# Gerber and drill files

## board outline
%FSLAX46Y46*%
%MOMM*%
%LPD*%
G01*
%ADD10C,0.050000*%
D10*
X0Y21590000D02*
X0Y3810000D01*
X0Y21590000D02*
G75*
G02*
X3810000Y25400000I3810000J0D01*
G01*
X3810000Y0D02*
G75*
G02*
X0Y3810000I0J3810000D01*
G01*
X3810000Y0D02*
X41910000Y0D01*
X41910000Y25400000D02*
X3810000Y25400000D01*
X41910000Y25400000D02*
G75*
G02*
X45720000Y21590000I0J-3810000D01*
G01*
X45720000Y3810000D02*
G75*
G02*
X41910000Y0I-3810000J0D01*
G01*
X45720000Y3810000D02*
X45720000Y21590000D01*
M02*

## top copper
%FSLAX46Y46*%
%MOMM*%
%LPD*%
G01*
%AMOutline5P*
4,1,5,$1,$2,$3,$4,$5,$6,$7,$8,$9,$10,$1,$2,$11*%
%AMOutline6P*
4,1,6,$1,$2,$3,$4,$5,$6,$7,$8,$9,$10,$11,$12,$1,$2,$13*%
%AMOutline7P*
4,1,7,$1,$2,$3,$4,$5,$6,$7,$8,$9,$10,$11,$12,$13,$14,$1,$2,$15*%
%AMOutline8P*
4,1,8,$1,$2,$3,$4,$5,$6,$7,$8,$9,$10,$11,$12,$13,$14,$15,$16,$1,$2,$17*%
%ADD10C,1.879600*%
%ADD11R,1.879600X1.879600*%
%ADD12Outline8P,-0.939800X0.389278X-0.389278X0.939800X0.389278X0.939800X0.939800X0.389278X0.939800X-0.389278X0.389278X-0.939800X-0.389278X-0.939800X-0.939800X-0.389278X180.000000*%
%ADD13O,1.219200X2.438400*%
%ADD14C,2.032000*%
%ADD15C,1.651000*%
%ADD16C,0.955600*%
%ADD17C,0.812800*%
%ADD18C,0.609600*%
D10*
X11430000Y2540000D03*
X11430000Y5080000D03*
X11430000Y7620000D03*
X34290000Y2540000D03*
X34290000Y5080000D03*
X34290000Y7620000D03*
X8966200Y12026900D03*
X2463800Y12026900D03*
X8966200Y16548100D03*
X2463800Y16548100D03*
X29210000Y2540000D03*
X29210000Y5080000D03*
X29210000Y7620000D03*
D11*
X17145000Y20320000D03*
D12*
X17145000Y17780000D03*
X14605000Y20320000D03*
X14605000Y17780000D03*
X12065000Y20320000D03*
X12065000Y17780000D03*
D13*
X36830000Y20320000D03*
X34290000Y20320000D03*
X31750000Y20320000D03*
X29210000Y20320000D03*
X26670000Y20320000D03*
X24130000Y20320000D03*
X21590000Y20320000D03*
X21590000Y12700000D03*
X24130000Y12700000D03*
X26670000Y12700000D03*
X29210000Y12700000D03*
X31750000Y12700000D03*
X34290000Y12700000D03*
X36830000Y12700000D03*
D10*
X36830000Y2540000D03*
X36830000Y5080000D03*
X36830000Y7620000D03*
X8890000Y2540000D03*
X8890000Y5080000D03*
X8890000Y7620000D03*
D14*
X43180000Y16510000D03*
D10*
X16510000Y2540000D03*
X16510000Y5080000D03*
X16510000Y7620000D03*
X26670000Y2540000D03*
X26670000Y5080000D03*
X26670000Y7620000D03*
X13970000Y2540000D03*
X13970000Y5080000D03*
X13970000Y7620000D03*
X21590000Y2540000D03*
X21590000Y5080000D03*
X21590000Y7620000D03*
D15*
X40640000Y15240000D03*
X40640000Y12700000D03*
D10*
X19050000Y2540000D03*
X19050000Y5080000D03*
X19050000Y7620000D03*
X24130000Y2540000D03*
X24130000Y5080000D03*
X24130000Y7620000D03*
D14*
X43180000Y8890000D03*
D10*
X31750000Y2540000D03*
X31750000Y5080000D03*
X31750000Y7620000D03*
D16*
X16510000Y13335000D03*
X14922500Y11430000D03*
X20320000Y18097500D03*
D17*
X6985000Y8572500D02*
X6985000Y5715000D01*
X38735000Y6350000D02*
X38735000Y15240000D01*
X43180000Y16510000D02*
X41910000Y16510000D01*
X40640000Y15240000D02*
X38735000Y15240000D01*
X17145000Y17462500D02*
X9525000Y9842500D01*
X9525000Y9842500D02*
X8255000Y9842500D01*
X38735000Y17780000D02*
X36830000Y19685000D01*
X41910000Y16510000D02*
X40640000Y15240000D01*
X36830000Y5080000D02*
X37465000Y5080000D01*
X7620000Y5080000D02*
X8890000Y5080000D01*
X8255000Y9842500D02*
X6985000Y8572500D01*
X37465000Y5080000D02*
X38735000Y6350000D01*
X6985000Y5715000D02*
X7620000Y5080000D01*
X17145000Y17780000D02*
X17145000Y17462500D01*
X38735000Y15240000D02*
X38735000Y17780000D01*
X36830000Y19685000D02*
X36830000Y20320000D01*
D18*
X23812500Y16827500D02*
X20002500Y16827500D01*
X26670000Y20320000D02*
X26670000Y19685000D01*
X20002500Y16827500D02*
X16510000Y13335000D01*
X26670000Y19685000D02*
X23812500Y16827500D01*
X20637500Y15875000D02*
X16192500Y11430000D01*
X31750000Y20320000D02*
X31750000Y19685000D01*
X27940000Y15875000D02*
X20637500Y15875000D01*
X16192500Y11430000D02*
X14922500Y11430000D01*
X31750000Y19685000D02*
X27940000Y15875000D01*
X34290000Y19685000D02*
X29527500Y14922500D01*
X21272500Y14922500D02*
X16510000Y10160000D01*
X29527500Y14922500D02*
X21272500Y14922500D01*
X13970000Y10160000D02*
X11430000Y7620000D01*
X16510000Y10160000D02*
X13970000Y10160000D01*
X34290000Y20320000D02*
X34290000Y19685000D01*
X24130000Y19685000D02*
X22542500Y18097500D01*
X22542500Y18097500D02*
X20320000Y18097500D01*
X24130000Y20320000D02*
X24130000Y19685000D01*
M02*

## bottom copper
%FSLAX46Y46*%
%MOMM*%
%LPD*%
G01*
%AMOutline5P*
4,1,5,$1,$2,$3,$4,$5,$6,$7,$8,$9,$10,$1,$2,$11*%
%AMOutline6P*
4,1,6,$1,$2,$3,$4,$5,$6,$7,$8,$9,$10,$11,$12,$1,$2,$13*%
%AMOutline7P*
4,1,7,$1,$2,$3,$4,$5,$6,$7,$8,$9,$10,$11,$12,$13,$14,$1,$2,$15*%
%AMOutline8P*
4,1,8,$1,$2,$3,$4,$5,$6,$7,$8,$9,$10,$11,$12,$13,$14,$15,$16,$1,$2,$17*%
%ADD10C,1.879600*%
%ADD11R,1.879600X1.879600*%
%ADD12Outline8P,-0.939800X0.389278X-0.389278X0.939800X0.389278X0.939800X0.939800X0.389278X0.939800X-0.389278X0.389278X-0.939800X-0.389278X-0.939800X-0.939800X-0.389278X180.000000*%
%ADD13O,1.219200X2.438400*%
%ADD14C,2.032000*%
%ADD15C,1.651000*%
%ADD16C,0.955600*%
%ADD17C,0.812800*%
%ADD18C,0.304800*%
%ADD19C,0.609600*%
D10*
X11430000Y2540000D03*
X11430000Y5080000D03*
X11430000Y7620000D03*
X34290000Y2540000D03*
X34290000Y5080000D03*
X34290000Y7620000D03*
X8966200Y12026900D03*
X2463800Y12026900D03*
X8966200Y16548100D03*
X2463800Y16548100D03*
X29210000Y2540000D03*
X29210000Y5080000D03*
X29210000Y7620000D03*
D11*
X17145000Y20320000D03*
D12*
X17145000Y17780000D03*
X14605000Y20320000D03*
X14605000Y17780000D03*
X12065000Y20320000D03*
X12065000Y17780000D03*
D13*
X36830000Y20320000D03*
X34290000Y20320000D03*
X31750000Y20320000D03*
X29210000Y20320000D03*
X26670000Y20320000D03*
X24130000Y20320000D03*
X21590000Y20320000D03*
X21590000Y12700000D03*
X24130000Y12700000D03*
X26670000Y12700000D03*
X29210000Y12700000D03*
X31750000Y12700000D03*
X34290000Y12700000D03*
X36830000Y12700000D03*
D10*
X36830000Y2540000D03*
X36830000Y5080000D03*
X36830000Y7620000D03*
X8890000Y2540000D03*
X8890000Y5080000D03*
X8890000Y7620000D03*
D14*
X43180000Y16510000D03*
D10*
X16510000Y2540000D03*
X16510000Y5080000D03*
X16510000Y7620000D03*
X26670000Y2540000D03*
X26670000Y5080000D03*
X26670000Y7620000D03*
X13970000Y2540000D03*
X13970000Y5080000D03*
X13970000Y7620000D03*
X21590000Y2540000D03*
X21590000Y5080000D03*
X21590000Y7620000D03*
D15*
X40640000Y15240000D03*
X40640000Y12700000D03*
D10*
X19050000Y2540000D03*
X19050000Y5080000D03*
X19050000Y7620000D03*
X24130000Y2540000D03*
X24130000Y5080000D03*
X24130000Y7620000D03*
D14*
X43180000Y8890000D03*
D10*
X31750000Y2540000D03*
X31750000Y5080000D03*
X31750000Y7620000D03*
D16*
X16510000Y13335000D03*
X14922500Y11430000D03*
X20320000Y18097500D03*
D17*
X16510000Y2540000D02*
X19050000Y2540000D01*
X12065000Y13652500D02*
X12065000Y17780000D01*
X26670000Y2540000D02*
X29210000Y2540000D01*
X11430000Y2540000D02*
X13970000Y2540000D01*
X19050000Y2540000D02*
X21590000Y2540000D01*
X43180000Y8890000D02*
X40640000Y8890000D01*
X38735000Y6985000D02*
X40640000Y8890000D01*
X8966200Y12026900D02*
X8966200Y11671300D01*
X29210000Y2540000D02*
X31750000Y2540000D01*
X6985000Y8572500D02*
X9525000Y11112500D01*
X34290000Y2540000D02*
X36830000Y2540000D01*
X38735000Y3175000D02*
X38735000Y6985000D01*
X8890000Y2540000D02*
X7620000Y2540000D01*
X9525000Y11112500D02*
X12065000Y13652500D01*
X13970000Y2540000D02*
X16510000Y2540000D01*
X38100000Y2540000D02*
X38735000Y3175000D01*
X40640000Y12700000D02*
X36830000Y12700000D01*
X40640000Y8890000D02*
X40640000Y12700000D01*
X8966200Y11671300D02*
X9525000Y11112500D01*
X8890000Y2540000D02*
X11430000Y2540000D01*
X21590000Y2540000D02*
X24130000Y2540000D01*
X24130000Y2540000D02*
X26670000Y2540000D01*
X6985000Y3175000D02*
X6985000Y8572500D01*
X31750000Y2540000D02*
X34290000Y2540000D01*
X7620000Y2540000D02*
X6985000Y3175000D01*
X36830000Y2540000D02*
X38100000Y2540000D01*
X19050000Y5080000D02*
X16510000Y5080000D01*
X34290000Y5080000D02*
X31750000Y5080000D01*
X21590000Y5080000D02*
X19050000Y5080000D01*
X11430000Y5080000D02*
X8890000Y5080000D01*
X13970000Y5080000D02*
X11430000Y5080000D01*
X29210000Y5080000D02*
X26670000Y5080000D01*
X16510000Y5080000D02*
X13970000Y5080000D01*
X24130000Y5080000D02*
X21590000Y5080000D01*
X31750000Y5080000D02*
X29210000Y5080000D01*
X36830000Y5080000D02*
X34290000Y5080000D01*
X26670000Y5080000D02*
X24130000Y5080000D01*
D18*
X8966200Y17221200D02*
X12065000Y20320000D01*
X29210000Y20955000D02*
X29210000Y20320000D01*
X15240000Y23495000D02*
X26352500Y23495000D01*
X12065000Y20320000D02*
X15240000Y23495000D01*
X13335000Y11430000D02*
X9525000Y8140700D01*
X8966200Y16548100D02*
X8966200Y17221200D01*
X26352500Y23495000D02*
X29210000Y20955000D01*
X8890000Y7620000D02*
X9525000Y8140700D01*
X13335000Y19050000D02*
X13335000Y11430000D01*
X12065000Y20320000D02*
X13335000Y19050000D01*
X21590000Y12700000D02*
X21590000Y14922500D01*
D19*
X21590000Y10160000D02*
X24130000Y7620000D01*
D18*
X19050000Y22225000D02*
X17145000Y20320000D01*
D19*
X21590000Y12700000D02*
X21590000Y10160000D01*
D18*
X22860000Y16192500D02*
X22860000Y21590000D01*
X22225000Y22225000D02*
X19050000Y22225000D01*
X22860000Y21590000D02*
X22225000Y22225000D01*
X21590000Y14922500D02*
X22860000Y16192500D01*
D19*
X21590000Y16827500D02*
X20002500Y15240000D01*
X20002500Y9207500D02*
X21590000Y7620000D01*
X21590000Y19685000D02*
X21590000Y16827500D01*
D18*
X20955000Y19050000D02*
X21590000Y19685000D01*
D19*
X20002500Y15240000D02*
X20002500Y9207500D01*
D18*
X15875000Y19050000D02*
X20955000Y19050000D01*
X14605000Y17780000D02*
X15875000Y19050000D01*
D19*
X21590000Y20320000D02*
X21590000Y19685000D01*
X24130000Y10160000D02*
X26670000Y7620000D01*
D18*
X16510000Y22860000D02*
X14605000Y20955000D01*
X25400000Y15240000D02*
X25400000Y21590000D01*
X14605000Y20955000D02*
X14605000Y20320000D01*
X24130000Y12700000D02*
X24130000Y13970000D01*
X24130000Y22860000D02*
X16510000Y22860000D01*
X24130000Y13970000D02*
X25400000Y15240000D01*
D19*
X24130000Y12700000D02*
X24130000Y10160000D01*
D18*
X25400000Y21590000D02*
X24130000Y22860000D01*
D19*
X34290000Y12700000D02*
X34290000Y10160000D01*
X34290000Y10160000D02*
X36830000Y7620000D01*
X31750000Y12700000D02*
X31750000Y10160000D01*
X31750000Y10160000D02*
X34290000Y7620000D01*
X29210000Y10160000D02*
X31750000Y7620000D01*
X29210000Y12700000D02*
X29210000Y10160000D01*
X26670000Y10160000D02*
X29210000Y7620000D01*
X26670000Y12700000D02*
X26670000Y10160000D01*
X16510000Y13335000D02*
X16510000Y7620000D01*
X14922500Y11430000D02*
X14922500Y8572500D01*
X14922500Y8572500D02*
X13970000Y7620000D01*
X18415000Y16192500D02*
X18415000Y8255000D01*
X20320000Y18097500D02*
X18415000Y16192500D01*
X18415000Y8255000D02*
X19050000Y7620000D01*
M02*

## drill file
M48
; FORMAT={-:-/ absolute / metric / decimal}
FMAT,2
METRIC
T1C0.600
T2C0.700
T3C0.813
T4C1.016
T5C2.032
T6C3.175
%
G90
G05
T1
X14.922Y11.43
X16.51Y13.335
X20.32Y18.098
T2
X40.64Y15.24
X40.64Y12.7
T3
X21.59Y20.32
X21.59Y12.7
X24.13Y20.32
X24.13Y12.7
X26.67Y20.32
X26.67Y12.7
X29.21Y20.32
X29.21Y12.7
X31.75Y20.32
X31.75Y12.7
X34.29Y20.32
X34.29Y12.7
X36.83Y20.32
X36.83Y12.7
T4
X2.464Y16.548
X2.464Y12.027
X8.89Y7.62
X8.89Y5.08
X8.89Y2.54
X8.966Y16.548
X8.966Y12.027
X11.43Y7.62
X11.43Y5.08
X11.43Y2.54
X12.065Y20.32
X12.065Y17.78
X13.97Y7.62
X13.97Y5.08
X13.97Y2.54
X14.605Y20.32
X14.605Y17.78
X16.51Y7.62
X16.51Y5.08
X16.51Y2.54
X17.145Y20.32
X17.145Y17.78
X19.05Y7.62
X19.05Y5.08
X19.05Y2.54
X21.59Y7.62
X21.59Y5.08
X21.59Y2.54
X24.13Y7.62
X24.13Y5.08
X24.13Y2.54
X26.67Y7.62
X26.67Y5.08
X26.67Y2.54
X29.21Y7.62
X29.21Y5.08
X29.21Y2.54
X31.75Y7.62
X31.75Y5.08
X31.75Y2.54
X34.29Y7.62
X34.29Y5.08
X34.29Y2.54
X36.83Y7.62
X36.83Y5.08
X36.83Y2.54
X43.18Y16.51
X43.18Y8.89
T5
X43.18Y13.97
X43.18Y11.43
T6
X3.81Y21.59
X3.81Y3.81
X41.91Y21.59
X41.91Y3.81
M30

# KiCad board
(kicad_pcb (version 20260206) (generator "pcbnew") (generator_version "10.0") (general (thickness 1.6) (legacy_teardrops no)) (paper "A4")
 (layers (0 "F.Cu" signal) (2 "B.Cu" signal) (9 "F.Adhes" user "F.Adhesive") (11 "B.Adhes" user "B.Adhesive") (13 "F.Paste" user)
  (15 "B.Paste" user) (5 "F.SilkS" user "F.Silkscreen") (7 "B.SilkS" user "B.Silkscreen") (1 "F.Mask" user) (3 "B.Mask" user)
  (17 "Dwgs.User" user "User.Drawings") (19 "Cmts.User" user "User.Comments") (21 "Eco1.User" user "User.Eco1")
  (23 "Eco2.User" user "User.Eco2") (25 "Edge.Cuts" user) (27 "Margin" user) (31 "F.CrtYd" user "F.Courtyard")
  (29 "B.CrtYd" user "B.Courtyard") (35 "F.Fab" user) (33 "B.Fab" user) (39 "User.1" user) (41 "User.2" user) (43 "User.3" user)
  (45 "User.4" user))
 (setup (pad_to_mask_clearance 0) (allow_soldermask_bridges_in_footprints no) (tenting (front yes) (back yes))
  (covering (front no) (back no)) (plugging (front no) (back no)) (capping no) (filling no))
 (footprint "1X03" (layer "F.Cu") (at 11.43 -2.54 90)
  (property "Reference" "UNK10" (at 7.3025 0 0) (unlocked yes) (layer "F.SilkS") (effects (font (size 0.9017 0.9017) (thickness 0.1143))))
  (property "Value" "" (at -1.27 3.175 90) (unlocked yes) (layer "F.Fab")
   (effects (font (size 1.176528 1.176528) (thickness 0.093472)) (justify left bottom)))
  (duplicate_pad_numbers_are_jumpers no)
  (pad "1" thru_hole circle (at 0 0 180) (size 1.8796 1.8796) (drill 1.016) (layers "*.Cu" "*.Mask") (remove_unused_layers no) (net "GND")
   (solder_mask_margin 0.0762) (thermal_bridge_angle 0))
  (pad "2" thru_hole circle (at 2.54 0 180) (size 1.8796 1.8796) (drill 1.016) (layers "*.Cu" "*.Mask") (remove_unused_layers no)
   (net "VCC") (solder_mask_margin 0.0762) (thermal_bridge_angle 0))
  (pad "3" thru_hole circle (at 5.08 0 180) (size 1.8796 1.8796) (drill 1.016) (layers "*.Cu" "*.Mask") (remove_unused_layers no)
   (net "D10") (solder_mask_margin 0.0762) (thermal_bridge_angle 0)))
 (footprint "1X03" (layer "F.Cu") (at 34.29 -2.54 90)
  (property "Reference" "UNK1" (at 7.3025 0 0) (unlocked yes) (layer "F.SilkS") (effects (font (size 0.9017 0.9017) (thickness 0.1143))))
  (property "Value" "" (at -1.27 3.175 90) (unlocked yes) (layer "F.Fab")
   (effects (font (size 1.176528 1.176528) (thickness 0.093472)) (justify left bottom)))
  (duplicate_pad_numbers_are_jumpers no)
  (pad "1" thru_hole circle (at 0 0 180) (size 1.8796 1.8796) (drill 1.016) (layers "*.Cu" "*.Mask") (remove_unused_layers no) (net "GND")
   (solder_mask_margin 0.0762) (thermal_bridge_angle 0))
  (pad "2" thru_hole circle (at 2.54 0 180) (size 1.8796 1.8796) (drill 1.016) (layers "*.Cu" "*.Mask") (remove_unused_layers no)
   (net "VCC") (solder_mask_margin 0.0762) (thermal_bridge_angle 0))
  (pad "3" thru_hole circle (at 5.08 0 180) (size 1.8796 1.8796) (drill 1.016) (layers "*.Cu" "*.Mask") (remove_unused_layers no) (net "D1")
   (solder_mask_margin 0.0762) (thermal_bridge_angle 0)))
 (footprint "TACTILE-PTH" (layer "F.Cu") (at 5.715 -14.2875 180)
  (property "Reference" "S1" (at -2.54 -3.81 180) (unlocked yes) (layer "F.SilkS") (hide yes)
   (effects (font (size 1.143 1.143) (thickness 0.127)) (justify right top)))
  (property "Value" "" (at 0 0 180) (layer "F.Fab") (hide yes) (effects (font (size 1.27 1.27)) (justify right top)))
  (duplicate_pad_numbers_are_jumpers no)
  (pad "1" thru_hole circle (at -3.2512 -2.2606 180) (size 1.8796 1.8796) (drill 1.016) (layers "*.Cu" "*.Mask") (remove_unused_layers no)
   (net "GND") (solder_mask_margin 0.0762) (thermal_bridge_angle 0))
  (pad "2" thru_hole circle (at 3.2512 -2.2606 180) (size 1.8796 1.8796) (drill 1.016) (layers "*.Cu" "*.Mask") (remove_unused_layers no)
   (solder_mask_margin 0.0762) (thermal_bridge_angle 0))
  (pad "3" thru_hole circle (at -3.2512 2.2606 180) (size 1.8796 1.8796) (drill 1.016) (layers "*.Cu" "*.Mask") (remove_unused_layers no)
   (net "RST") (solder_mask_margin 0.0762) (thermal_bridge_angle 0))
  (pad "4" thru_hole circle (at 3.2512 2.2606 180) (size 1.8796 1.8796) (drill 1.016) (layers "*.Cu" "*.Mask") (remove_unused_layers no)
   (solder_mask_margin 0.0762) (thermal_bridge_angle 0)))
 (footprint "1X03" (layer "F.Cu") (at 29.21 -2.54 90)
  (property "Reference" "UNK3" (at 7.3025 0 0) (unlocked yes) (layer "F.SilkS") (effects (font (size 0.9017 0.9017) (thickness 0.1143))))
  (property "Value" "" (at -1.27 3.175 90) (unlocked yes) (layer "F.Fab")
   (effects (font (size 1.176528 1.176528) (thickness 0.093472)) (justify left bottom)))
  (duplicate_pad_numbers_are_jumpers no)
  (pad "1" thru_hole circle (at 0 0 180) (size 1.8796 1.8796) (drill 1.016) (layers "*.Cu" "*.Mask") (remove_unused_layers no) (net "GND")
   (solder_mask_margin 0.0762) (thermal_bridge_angle 0))
  (pad "2" thru_hole circle (at 2.54 0 180) (size 1.8796 1.8796) (drill 1.016) (layers "*.Cu" "*.Mask") (remove_unused_layers no)
   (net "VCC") (solder_mask_margin 0.0762) (thermal_bridge_angle 0))
  (pad "3" thru_hole circle (at 5.08 0 180) (size 1.8796 1.8796) (drill 1.016) (layers "*.Cu" "*.Mask") (remove_unused_layers no) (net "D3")
   (solder_mask_margin 0.0762) (thermal_bridge_angle 0)))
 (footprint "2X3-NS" (layer "F.Cu") (at 14.605 -19.05 180)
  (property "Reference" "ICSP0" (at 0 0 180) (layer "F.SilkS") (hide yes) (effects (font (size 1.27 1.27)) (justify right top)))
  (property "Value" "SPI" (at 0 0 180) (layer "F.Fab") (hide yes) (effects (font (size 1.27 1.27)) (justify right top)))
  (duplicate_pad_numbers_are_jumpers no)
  (pad "1" thru_hole rect (at -2.54 1.27 180) (size 1.8796 1.8796) (drill 1.016) (layers "*.Cu" "*.Mask") (remove_unused_layers no)
   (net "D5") (solder_mask_margin 0.0762) (thermal_bridge_angle 0))
  (pad "2" thru_hole roundrect (at -2.54 -1.27 180) (size 1.8796 1.8796) (drill 1.016) (layers "*.Cu" "*.Mask") (remove_unused_layers no)
   (roundrect_rratio 0.25) (chamfer_ratio 0.2928932188) (chamfer top_left top_right bottom_left bottom_right) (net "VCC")
   (solder_mask_margin 0.0762) (thermal_bridge_angle 0))
  (pad "3" thru_hole roundrect (at 0 1.27 180) (size 1.8796 1.8796) (drill 1.016) (layers "*.Cu" "*.Mask") (remove_unused_layers no)
   (roundrect_rratio 0.25) (chamfer_ratio 0.2928932188) (chamfer top_left top_right bottom_left bottom_right) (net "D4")
   (solder_mask_margin 0.0762) (thermal_bridge_angle 0))
  (pad "4" thru_hole roundrect (at 0 -1.27 180) (size 1.8796 1.8796) (drill 1.016) (layers "*.Cu" "*.Mask") (remove_unused_layers no)
   (roundrect_rratio 0.25) (chamfer_ratio 0.2928932188) (chamfer top_left top_right bottom_left bottom_right) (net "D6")
   (solder_mask_margin 0.0762) (thermal_bridge_angle 0))
  (pad "5" thru_hole roundrect (at 2.54 1.27 180) (size 1.8796 1.8796) (drill 1.016) (layers "*.Cu" "*.Mask") (remove_unused_layers no)
   (roundrect_rratio 0.25) (chamfer_ratio 0.2928932188) (chamfer top_left top_right bottom_left bottom_right) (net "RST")
   (solder_mask_margin 0.0762) (thermal_bridge_angle 0))
  (pad "6" thru_hole roundrect (at 2.54 -1.27 180) (size 1.8796 1.8796) (drill 1.016) (layers "*.Cu" "*.Mask") (remove_unused_layers no)
   (roundrect_rratio 0.25) (chamfer_ratio 0.2928932188) (chamfer top_left top_right bottom_left bottom_right) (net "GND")
   (solder_mask_margin 0.0762) (thermal_bridge_angle 0)))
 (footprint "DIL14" (layer "F.Cu") (at 27.94 -16.51 180)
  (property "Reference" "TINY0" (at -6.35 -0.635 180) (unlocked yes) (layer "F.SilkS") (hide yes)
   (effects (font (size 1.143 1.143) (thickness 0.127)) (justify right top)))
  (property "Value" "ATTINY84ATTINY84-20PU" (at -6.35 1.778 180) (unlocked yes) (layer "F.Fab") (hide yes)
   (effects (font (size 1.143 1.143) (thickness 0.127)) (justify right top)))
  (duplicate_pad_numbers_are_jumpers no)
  (pad "1" thru_hole oval (at -8.89 3.81 270) (size 2.4384 1.2192) (drill 0.8128) (layers "*.Cu" "*.Mask") (remove_unused_layers no)
   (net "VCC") (solder_mask_margin 0.0762) (thermal_bridge_angle 0))
  (pad "2" thru_hole oval (at -6.35 3.81 270) (size 2.4384 1.2192) (drill 0.8128) (layers "*.Cu" "*.Mask") (remove_unused_layers no)
   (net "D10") (solder_mask_margin 0.0762) (thermal_bridge_angle 0))
  (pad "3" thru_hole oval (at -3.81 3.81 270) (size 2.4384 1.2192) (drill 0.8128) (layers "*.Cu" "*.Mask") (remove_unused_layers no)
   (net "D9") (solder_mask_margin 0.0762) (thermal_bridge_angle 0))
  (pad "4" thru_hole oval (at -1.27 3.81 270) (size 2.4384 1.2192) (drill 0.8128) (layers "*.Cu" "*.Mask") (remove_unused_layers no)
   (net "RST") (solder_mask_margin 0.0762) (thermal_bridge_angle 0))
  (pad "5" thru_hole oval (at 1.27 3.81 270) (size 2.4384 1.2192) (drill 0.8128) (layers "*.Cu" "*.Mask") (remove_unused_layers no)
   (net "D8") (solder_mask_margin 0.0762) (thermal_bridge_angle 0))
  (pad "6" thru_hole oval (at 3.81 3.81 270) (size 2.4384 1.2192) (drill 0.8128) (layers "*.Cu" "*.Mask") (remove_unused_layers no)
   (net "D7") (solder_mask_margin 0.0762) (thermal_bridge_angle 0))
  (pad "7" thru_hole oval (at 6.35 3.81 270) (size 2.4384 1.2192) (drill 0.8128) (layers "*.Cu" "*.Mask") (remove_unused_layers no)
   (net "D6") (solder_mask_margin 0.0762) (thermal_bridge_angle 0))
  (pad "8" thru_hole oval (at 6.35 -3.81 270) (size 2.4384 1.2192) (drill 0.8128) (layers "*.Cu" "*.Mask") (remove_unused_layers no)
   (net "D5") (solder_mask_margin 0.0762) (thermal_bridge_angle 0))
  (pad "9" thru_hole oval (at 3.81 -3.81 270) (size 2.4384 1.2192) (drill 0.8128) (layers "*.Cu" "*.Mask") (remove_unused_layers no)
   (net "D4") (solder_mask_margin 0.0762) (thermal_bridge_angle 0))
  (pad "10" thru_hole oval (at 1.27 -3.81 270) (size 2.4384 1.2192) (drill 0.8128) (layers "*.Cu" "*.Mask") (remove_unused_layers no)
   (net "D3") (solder_mask_margin 0.0762) (thermal_bridge_angle 0))
  (pad "11" thru_hole oval (at -1.27 -3.81 270) (size 2.4384 1.2192) (drill 0.8128) (layers "*.Cu" "*.Mask") (remove_unused_layers no)
   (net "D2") (solder_mask_margin 0.0762) (thermal_bridge_angle 0))
  (pad "12" thru_hole oval (at -3.81 -3.81 270) (size 2.4384 1.2192) (drill 0.8128) (layers "*.Cu" "*.Mask") (remove_unused_layers no)
   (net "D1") (solder_mask_margin 0.0762) (thermal_bridge_angle 0))
  (pad "13" thru_hole oval (at -6.35 -3.81 270) (size 2.4384 1.2192) (drill 0.8128) (layers "*.Cu" "*.Mask") (remove_unused_layers no)
   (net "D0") (solder_mask_margin 0.0762) (thermal_bridge_angle 0))
  (pad "14" thru_hole oval (at -8.89 -3.81 270) (size 2.4384 1.2192) (drill 0.8128) (layers "*.Cu" "*.Mask") (remove_unused_layers no)
   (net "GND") (solder_mask_margin 0.0762) (thermal_bridge_angle 0)))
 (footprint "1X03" (layer "F.Cu") (at 36.83 -2.54 90)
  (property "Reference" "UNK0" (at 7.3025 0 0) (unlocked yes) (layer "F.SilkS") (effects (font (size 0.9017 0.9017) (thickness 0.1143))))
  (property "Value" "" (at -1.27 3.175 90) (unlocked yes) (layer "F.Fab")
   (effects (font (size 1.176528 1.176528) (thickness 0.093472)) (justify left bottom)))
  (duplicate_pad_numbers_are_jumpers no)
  (pad "1" thru_hole circle (at 0 0 180) (size 1.8796 1.8796) (drill 1.016) (layers "*.Cu" "*.Mask") (remove_unused_layers no) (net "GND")
   (solder_mask_margin 0.0762) (thermal_bridge_angle 0))
  (pad "2" thru_hole circle (at 2.54 0 180) (size 1.8796 1.8796) (drill 1.016) (layers "*.Cu" "*.Mask") (remove_unused_layers no)
   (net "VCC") (solder_mask_margin 0.0762) (thermal_bridge_angle 0))
  (pad "3" thru_hole circle (at 5.08 0 180) (size 1.8796 1.8796) (drill 1.016) (layers "*.Cu" "*.Mask") (remove_unused_layers no) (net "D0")
   (solder_mask_margin 0.0762) (thermal_bridge_angle 0)))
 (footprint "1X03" (layer "F.Cu") (at 8.89 -2.54 90)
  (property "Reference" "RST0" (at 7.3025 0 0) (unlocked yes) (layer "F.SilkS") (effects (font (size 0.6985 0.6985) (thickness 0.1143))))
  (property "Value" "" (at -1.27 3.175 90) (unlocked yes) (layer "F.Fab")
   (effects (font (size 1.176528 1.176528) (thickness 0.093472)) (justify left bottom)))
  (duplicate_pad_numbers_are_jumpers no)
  (pad "1" thru_hole circle (at 0 0 180) (size 1.8796 1.8796) (drill 1.016) (layers "*.Cu" "*.Mask") (remove_unused_layers no) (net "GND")
   (solder_mask_margin 0.0762) (thermal_bridge_angle 0))
  (pad "2" thru_hole circle (at 2.54 0 180) (size 1.8796 1.8796) (drill 1.016) (layers "*.Cu" "*.Mask") (remove_unused_layers no)
   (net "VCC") (solder_mask_margin 0.0762) (thermal_bridge_angle 0))
  (pad "3" thru_hole circle (at 5.08 0 180) (size 1.8796 1.8796) (drill 1.016) (layers "*.Cu" "*.Mask") (remove_unused_layers no)
   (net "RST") (solder_mask_margin 0.0762) (thermal_bridge_angle 0)))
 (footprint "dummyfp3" (layer "F.Cu") (at 41.91 -21.59)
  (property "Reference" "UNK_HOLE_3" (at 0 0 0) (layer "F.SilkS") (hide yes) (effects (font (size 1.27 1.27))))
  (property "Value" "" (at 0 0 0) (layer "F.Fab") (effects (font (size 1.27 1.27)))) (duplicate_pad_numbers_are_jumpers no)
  (pad "" np_thru_hole circle (at 0 0) (size 3.175 3.175) (drill 3.175) (layers "*.Cu" "*.Mask")))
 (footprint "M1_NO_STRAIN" (layer "F.Cu") (at 43.18 -16.51 -90)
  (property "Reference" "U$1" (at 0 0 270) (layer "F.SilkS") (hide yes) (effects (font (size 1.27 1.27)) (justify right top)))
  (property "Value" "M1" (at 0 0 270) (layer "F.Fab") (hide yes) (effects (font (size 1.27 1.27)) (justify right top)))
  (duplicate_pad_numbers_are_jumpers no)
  (pad "" np_thru_hole circle (at 2.54 0 270) (size 2.032 2.032) (drill 2.032) (layers "*.Cu" "*.Mask"))
  (pad "P$1" thru_hole circle (at 0 0 270) (size 2.032 2.032) (drill 1.016) (layers "*.Cu" "*.Mask") (remove_unused_layers no) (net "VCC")
   (solder_mask_margin 0.0762) (thermal_bridge_angle 0)))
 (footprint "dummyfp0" (layer "F.Cu") (at 3.81 -3.81)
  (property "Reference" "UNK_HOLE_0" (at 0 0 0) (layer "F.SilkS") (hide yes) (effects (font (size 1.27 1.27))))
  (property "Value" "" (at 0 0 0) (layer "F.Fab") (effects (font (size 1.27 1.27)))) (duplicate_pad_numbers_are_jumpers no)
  (pad "" np_thru_hole circle (at 0 0) (size 3.175 3.175) (drill 3.175) (layers "*.Cu" "*.Mask")))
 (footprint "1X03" (layer "F.Cu") (at 16.51 -2.54 90)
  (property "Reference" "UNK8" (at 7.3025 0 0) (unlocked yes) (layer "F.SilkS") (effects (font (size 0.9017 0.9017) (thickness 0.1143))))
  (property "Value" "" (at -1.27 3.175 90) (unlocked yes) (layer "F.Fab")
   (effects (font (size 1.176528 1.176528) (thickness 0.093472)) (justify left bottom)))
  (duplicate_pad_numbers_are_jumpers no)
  (pad "1" thru_hole circle (at 0 0 180) (size 1.8796 1.8796) (drill 1.016) (layers "*.Cu" "*.Mask") (remove_unused_layers no) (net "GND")
   (solder_mask_margin 0.0762) (thermal_bridge_angle 0))
  (pad "2" thru_hole circle (at 2.54 0 180) (size 1.8796 1.8796) (drill 1.016) (layers "*.Cu" "*.Mask") (remove_unused_layers no)
   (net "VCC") (solder_mask_margin 0.0762) (thermal_bridge_angle 0))
  (pad "3" thru_hole circle (at 5.08 0 180) (size 1.8796 1.8796) (drill 1.016) (layers "*.Cu" "*.Mask") (remove_unused_layers no) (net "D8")
   (solder_mask_margin 0.0762) (thermal_bridge_angle 0)))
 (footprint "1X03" (layer "F.Cu") (at 26.67 -2.54 90)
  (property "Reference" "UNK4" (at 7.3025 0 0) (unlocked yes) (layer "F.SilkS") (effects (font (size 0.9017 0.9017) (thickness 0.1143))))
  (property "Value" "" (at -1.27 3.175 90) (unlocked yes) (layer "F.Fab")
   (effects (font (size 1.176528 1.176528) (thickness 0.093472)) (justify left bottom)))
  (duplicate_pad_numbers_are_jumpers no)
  (pad "1" thru_hole circle (at 0 0 180) (size 1.8796 1.8796) (drill 1.016) (layers "*.Cu" "*.Mask") (remove_unused_layers no) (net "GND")
   (solder_mask_margin 0.0762) (thermal_bridge_angle 0))
  (pad "2" thru_hole circle (at 2.54 0 180) (size 1.8796 1.8796) (drill 1.016) (layers "*.Cu" "*.Mask") (remove_unused_layers no)
   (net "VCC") (solder_mask_margin 0.0762) (thermal_bridge_angle 0))
  (pad "3" thru_hole circle (at 5.08 0 180) (size 1.8796 1.8796) (drill 1.016) (layers "*.Cu" "*.Mask") (remove_unused_layers no) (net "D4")
   (solder_mask_margin 0.0762) (thermal_bridge_angle 0)))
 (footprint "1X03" (layer "F.Cu") (at 13.97 -2.54 90)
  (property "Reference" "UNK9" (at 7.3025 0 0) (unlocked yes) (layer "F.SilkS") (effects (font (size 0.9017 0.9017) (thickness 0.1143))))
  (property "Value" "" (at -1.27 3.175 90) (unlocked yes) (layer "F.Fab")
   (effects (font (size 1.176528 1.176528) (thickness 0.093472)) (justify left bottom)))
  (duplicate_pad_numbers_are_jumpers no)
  (pad "1" thru_hole circle (at 0 0 180) (size 1.8796 1.8796) (drill 1.016) (layers "*.Cu" "*.Mask") (remove_unused_layers no) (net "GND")
   (solder_mask_margin 0.0762) (thermal_bridge_angle 0))
  (pad "2" thru_hole circle (at 2.54 0 180) (size 1.8796 1.8796) (drill 1.016) (layers "*.Cu" "*.Mask") (remove_unused_layers no)
   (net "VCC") (solder_mask_margin 0.0762) (thermal_bridge_angle 0))
  (pad "3" thru_hole circle (at 5.08 0 180) (size 1.8796 1.8796) (drill 1.016) (layers "*.Cu" "*.Mask") (remove_unused_layers no) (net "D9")
   (solder_mask_margin 0.0762) (thermal_bridge_angle 0)))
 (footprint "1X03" (layer "F.Cu") (at 21.59 -2.54 90)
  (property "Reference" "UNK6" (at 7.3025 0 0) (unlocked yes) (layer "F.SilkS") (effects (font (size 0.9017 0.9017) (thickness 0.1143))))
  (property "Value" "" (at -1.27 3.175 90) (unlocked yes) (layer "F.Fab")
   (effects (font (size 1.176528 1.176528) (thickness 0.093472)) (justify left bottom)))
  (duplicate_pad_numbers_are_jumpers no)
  (pad "1" thru_hole circle (at 0 0 180) (size 1.8796 1.8796) (drill 1.016) (layers "*.Cu" "*.Mask") (remove_unused_layers no) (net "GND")
   (solder_mask_margin 0.0762) (thermal_bridge_angle 0))
  (pad "2" thru_hole circle (at 2.54 0 180) (size 1.8796 1.8796) (drill 1.016) (layers "*.Cu" "*.Mask") (remove_unused_layers no)
   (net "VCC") (solder_mask_margin 0.0762) (thermal_bridge_angle 0))
  (pad "3" thru_hole circle (at 5.08 0 180) (size 1.8796 1.8796) (drill 1.016) (layers "*.Cu" "*.Mask") (remove_unused_layers no) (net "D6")
   (solder_mask_margin 0.0762) (thermal_bridge_angle 0)))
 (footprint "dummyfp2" (layer "F.Cu") (at 3.81 -21.59)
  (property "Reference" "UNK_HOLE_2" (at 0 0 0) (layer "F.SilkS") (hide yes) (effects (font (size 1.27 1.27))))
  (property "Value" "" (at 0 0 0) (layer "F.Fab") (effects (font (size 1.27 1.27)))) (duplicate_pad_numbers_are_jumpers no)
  (pad "" np_thru_hole circle (at 0 0) (size 3.175 3.175) (drill 3.175) (layers "*.Cu" "*.Mask")))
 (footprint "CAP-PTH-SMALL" (layer "F.Cu") (at 40.64 -15.24 -90)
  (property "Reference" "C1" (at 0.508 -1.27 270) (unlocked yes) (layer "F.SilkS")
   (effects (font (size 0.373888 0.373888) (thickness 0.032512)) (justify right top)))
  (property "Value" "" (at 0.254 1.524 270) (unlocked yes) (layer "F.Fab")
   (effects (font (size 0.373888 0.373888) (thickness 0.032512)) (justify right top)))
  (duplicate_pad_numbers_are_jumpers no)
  (pad "1" thru_hole circle (at 0 0 270) (size 1.651 1.651) (drill 0.7) (layers "*.Cu" "*.Mask") (remove_unused_layers no) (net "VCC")
   (solder_mask_margin 0.0762) (thermal_bridge_angle 0))
  (pad "2" thru_hole circle (at 2.54 0 270) (size 1.651 1.651) (drill 0.7) (layers "*.Cu" "*.Mask") (remove_unused_layers no) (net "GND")
   (solder_mask_margin 0.0762) (thermal_bridge_angle 0)))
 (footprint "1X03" (layer "F.Cu") (at 19.05 -2.54 90)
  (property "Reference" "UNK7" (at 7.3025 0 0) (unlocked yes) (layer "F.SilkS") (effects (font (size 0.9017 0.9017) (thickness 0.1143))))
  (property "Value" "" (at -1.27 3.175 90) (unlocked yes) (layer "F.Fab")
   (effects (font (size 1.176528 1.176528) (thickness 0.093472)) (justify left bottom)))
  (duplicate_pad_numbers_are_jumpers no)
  (pad "1" thru_hole circle (at 0 0 180) (size 1.8796 1.8796) (drill 1.016) (layers "*.Cu" "*.Mask") (remove_unused_layers no) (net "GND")
   (solder_mask_margin 0.0762) (thermal_bridge_angle 0))
  (pad "2" thru_hole circle (at 2.54 0 180) (size 1.8796 1.8796) (drill 1.016) (layers "*.Cu" "*.Mask") (remove_unused_layers no)
   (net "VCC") (solder_mask_margin 0.0762) (thermal_bridge_angle 0))
  (pad "3" thru_hole circle (at 5.08 0 180) (size 1.8796 1.8796) (drill 1.016) (layers "*.Cu" "*.Mask") (remove_unused_layers no) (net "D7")
   (solder_mask_margin 0.0762) (thermal_bridge_angle 0)))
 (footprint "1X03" (layer "F.Cu") (at 24.13 -2.54 90)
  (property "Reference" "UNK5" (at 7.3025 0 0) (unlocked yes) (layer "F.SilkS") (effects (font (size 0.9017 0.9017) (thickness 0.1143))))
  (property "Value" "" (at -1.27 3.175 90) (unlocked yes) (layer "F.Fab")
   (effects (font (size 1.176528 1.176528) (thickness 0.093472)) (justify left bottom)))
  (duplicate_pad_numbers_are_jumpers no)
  (pad "1" thru_hole circle (at 0 0 180) (size 1.8796 1.8796) (drill 1.016) (layers "*.Cu" "*.Mask") (remove_unused_layers no) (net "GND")
   (solder_mask_margin 0.0762) (thermal_bridge_angle 0))
  (pad "2" thru_hole circle (at 2.54 0 180) (size 1.8796 1.8796) (drill 1.016) (layers "*.Cu" "*.Mask") (remove_unused_layers no)
   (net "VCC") (solder_mask_margin 0.0762) (thermal_bridge_angle 0))
  (pad "3" thru_hole circle (at 5.08 0 180) (size 1.8796 1.8796) (drill 1.016) (layers "*.Cu" "*.Mask") (remove_unused_layers no) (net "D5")
   (solder_mask_margin 0.0762) (thermal_bridge_angle 0)))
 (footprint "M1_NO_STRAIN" (layer "F.Cu") (at 43.18 -8.89 90)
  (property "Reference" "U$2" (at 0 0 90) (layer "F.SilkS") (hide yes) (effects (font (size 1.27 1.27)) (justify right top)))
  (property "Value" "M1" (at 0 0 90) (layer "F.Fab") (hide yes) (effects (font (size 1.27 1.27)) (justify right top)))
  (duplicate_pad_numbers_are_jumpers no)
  (pad "" np_thru_hole circle (at 2.54 0 90) (size 2.032 2.032) (drill 2.032) (layers "*.Cu" "*.Mask"))
  (pad "P$1" thru_hole circle (at 0 0 90) (size 2.032 2.032) (drill 1.016) (layers "*.Cu" "*.Mask") (remove_unused_layers no) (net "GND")
   (solder_mask_margin 0.0762) (thermal_bridge_angle 0)))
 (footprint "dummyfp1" (layer "F.Cu") (at 41.91 -3.81)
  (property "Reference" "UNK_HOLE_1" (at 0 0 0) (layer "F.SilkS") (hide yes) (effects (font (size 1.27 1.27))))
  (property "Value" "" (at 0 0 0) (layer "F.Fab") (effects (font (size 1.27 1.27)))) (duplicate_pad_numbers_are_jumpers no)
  (pad "" np_thru_hole circle (at 0 0) (size 3.175 3.175) (drill 3.175) (layers "*.Cu" "*.Mask")))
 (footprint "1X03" (layer "F.Cu") (at 31.75 -2.54 90)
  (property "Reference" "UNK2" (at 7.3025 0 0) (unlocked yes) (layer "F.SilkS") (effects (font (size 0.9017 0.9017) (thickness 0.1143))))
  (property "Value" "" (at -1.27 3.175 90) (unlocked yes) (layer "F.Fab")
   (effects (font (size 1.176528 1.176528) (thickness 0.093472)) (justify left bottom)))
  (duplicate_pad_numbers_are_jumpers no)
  (pad "1" thru_hole circle (at 0 0 180) (size 1.8796 1.8796) (drill 1.016) (layers "*.Cu" "*.Mask") (remove_unused_layers no) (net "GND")
   (solder_mask_margin 0.0762) (thermal_bridge_angle 0))
  (pad "2" thru_hole circle (at 2.54 0 180) (size 1.8796 1.8796) (drill 1.016) (layers "*.Cu" "*.Mask") (remove_unused_layers no)
   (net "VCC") (solder_mask_margin 0.0762) (thermal_bridge_angle 0))
  (pad "3" thru_hole circle (at 5.08 0 180) (size 1.8796 1.8796) (drill 1.016) (layers "*.Cu" "*.Mask") (remove_unused_layers no) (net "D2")
   (solder_mask_margin 0.0762) (thermal_bridge_angle 0)))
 (gr_line (start 0 -21.59) (end 0 -3.81) (stroke (width 0.05) (type solid)) (layer "Edge.Cuts"))
 (gr_arc (start 0 -21.59) (mid 1.115923 -24.284077) (end 3.81 -25.4) (stroke (width 0.05) (type solid)) (layer "Edge.Cuts"))
 (gr_arc (start 3.81 0) (mid 1.115923 -1.115923) (end 0 -3.81) (stroke (width 0.05) (type solid)) (layer "Edge.Cuts"))
 (gr_line (start 3.81 0) (end 41.91 0) (stroke (width 0.05) (type solid)) (layer "Edge.Cuts"))
 (gr_line (start 41.91 -25.4) (end 3.81 -25.4) (stroke (width 0.05) (type solid)) (layer "Edge.Cuts"))
 (gr_arc (start 41.91 -25.4) (mid 44.604077 -24.284077) (end 45.72 -21.59) (stroke (width 0.05) (type solid)) (layer "Edge.Cuts"))
 (gr_arc (start 45.72 -3.81) (mid 44.604077 -1.115923) (end 41.91 0) (stroke (width 0.05) (type solid)) (layer "Edge.Cuts"))
 (gr_line (start 45.72 -3.81) (end 45.72 -21.59) (stroke (width 0.05) (type solid)) (layer "Edge.Cuts"))
 (segment (start 16.51 -2.54) (end 19.05 -2.54) (width 0.8128) (layer "B.Cu") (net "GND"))
 (segment (start 12.065 -13.6525) (end 12.065 -17.78) (width 0.8128) (layer "B.Cu") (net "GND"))
 (segment (start 26.67 -2.54) (end 29.21 -2.54) (width 0.8128) (layer "B.Cu") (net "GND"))
 (segment (start 11.43 -2.54) (end 13.97 -2.54) (width 0.8128) (layer "B.Cu") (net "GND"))
 (segment (start 19.05 -2.54) (end 21.59 -2.54) (width 0.8128) (layer "B.Cu") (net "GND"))
 (segment (start 43.18 -8.89) (end 40.64 -8.89) (width 0.8128) (layer "B.Cu") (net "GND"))
 (segment (start 38.735 -6.985) (end 40.64 -8.89) (width 0.8128) (layer "B.Cu") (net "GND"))
 (segment (start 8.9662 -12.0269) (end 8.9662 -11.6713) (width 0.8128) (layer "B.Cu") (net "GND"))
 (segment (start 29.21 -2.54) (end 31.75 -2.54) (width 0.8128) (layer "B.Cu") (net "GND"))
 (segment (start 6.985 -8.5725) (end 9.525 -11.1125) (width 0.8128) (layer "B.Cu") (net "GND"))
 (segment (start 34.29 -2.54) (end 36.83 -2.54) (width 0.8128) (layer "B.Cu") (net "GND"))
 (segment (start 38.735 -3.175) (end 38.735 -6.985) (width 0.8128) (layer "B.Cu") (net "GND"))
 (segment (start 8.89 -2.54) (end 7.62 -2.54) (width 0.8128) (layer "B.Cu") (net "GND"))
 (segment (start 9.525 -11.1125) (end 12.065 -13.6525) (width 0.8128) (layer "B.Cu") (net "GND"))
 (segment (start 13.97 -2.54) (end 16.51 -2.54) (width 0.8128) (layer "B.Cu") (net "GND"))
 (segment (start 38.1 -2.54) (end 38.735 -3.175) (width 0.8128) (layer "B.Cu") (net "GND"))
 (segment (start 40.64 -12.7) (end 36.83 -12.7) (width 0.8128) (layer "B.Cu") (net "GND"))
 (segment (start 40.64 -8.89) (end 40.64 -12.7) (width 0.8128) (layer "B.Cu") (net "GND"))
 (segment (start 8.9662 -11.6713) (end 9.525 -11.1125) (width 0.8128) (layer "B.Cu") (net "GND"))
 (segment (start 8.89 -2.54) (end 11.43 -2.54) (width 0.8128) (layer "B.Cu") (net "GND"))
 (segment (start 21.59 -2.54) (end 24.13 -2.54) (width 0.8128) (layer "B.Cu") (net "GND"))
 (segment (start 24.13 -2.54) (end 26.67 -2.54) (width 0.8128) (layer "B.Cu") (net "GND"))
 (segment (start 6.985 -3.175) (end 6.985 -8.5725) (width 0.8128) (layer "B.Cu") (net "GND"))
 (segment (start 31.75 -2.54) (end 34.29 -2.54) (width 0.8128) (layer "B.Cu") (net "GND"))
 (segment (start 7.62 -2.54) (end 6.985 -3.175) (width 0.8128) (layer "B.Cu") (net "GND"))
 (segment (start 36.83 -2.54) (end 38.1 -2.54) (width 0.8128) (layer "B.Cu") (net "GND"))
 (segment (start 6.985 -8.5725) (end 6.985 -5.715) (width 0.8128) (layer "F.Cu") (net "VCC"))
 (segment (start 38.735 -6.35) (end 38.735 -15.24) (width 0.8128) (layer "F.Cu") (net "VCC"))
 (segment (start 43.18 -16.51) (end 41.91 -16.51) (width 0.8128) (layer "F.Cu") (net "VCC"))
 (segment (start 40.64 -15.24) (end 38.735 -15.24) (width 0.8128) (layer "F.Cu") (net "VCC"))
 (segment (start 17.145 -17.4625) (end 9.525 -9.8425) (width 0.8128) (layer "F.Cu") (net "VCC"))
 (segment (start 9.525 -9.8425) (end 8.255 -9.8425) (width 0.8128) (layer "F.Cu") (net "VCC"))
 (segment (start 38.735 -17.78) (end 36.83 -19.685) (width 0.8128) (layer "F.Cu") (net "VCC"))
 (segment (start 41.91 -16.51) (end 40.64 -15.24) (width 0.8128) (layer "F.Cu") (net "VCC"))
 (segment (start 36.83 -5.08) (end 37.465 -5.08) (width 0.8128) (layer "F.Cu") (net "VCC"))
 (segment (start 7.62 -5.08) (end 8.89 -5.08) (width 0.8128) (layer "F.Cu") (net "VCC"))
 (segment (start 8.255 -9.8425) (end 6.985 -8.5725) (width 0.8128) (layer "F.Cu") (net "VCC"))
 (segment (start 37.465 -5.08) (end 38.735 -6.35) (width 0.8128) (layer "F.Cu") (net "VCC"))
 (segment (start 6.985 -5.715) (end 7.62 -5.08) (width 0.8128) (layer "F.Cu") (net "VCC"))
 (segment (start 17.145 -17.78) (end 17.145 -17.4625) (width 0.8128) (layer "F.Cu") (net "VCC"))
 (segment (start 38.735 -15.24) (end 38.735 -17.78) (width 0.8128) (layer "F.Cu") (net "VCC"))
 (segment (start 36.83 -19.685) (end 36.83 -20.32) (width 0.8128) (layer "F.Cu") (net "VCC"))
 (segment (start 19.05 -5.08) (end 16.51 -5.08) (width 0.8128) (layer "B.Cu") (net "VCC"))
 (segment (start 34.29 -5.08) (end 31.75 -5.08) (width 0.8128) (layer "B.Cu") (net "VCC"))
 (segment (start 21.59 -5.08) (end 19.05 -5.08) (width 0.8128) (layer "B.Cu") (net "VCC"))
 (segment (start 11.43 -5.08) (end 8.89 -5.08) (width 0.8128) (layer "B.Cu") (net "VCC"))
 (segment (start 13.97 -5.08) (end 11.43 -5.08) (width 0.8128) (layer "B.Cu") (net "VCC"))
 (segment (start 29.21 -5.08) (end 26.67 -5.08) (width 0.8128) (layer "B.Cu") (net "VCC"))
 (segment (start 16.51 -5.08) (end 13.97 -5.08) (width 0.8128) (layer "B.Cu") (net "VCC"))
 (segment (start 24.13 -5.08) (end 21.59 -5.08) (width 0.8128) (layer "B.Cu") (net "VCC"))
 (segment (start 31.75 -5.08) (end 29.21 -5.08) (width 0.8128) (layer "B.Cu") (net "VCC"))
 (segment (start 36.83 -5.08) (end 34.29 -5.08) (width 0.8128) (layer "B.Cu") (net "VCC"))
 (segment (start 26.67 -5.08) (end 24.13 -5.08) (width 0.8128) (layer "B.Cu") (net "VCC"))
 (segment (start 8.9662 -17.2212) (end 12.065 -20.32) (width 0.3048) (layer "B.Cu") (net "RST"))
 (segment (start 29.21 -20.955) (end 29.21 -20.32) (width 0.3048) (layer "B.Cu") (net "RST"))
 (segment (start 15.24 -23.495) (end 26.3525 -23.495) (width 0.3048) (layer "B.Cu") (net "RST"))
 (segment (start 12.065 -20.32) (end 15.24 -23.495) (width 0.3048) (layer "B.Cu") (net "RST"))
 (segment (start 13.335 -11.43) (end 9.525 -8.1407) (width 0.3048) (layer "B.Cu") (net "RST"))
 (segment (start 8.9662 -16.5481) (end 8.9662 -17.2212) (width 0.3048) (layer "B.Cu") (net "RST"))
 (segment (start 26.3525 -23.495) (end 29.21 -20.955) (width 0.3048) (layer "B.Cu") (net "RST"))
 (segment (start 8.89 -7.62) (end 9.525 -8.1407) (width 0.3048) (layer "B.Cu") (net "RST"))
 (segment (start 13.335 -19.05) (end 13.335 -11.43) (width 0.3048) (layer "B.Cu") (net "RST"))
 (segment (start 12.065 -20.32) (end 13.335 -19.05) (width 0.3048) (layer "B.Cu") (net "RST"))
 (segment (start 21.59 -12.7) (end 21.59 -14.9225) (width 0.3048) (layer "B.Cu") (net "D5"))
 (segment (start 21.59 -10.16) (end 24.13 -7.62) (width 0.6096) (layer "B.Cu") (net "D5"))
 (segment (start 19.05 -22.225) (end 17.145 -20.32) (width 0.3048) (layer "B.Cu") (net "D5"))
 (segment (start 21.59 -12.7) (end 21.59 -10.16) (width 0.6096) (layer "B.Cu") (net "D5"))
 (segment (start 22.86 -16.1925) (end 22.86 -21.59) (width 0.3048) (layer "B.Cu") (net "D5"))
 (segment (start 22.225 -22.225) (end 19.05 -22.225) (width 0.3048) (layer "B.Cu") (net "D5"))
 (segment (start 22.86 -21.59) (end 22.225 -22.225) (width 0.3048) (layer "B.Cu") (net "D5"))
 (segment (start 21.59 -14.9225) (end 22.86 -16.1925) (width 0.3048) (layer "B.Cu") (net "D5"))
 (segment (start 21.59 -16.8275) (end 20.0025 -15.24) (width 0.6096) (layer "B.Cu") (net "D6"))
 (segment (start 20.0025 -9.2075) (end 21.59 -7.62) (width 0.6096) (layer "B.Cu") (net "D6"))
 (segment (start 21.59 -19.685) (end 21.59 -16.8275) (width 0.6096) (layer "B.Cu") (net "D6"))
 (segment (start 20.955 -19.05) (end 21.59 -19.685) (width 0.3048) (layer "B.Cu") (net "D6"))
 (segment (start 20.0025 -15.24) (end 20.0025 -9.2075) (width 0.6096) (layer "B.Cu") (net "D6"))
 (segment (start 15.875 -19.05) (end 20.955 -19.05) (width 0.3048) (layer "B.Cu") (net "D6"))
 (segment (start 14.605 -17.78) (end 15.875 -19.05) (width 0.3048) (layer "B.Cu") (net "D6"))
 (segment (start 21.59 -20.32) (end 21.59 -19.685) (width 0.6096) (layer "B.Cu") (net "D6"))
 (segment (start 24.13 -10.16) (end 26.67 -7.62) (width 0.6096) (layer "B.Cu") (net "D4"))
 (segment (start 16.51 -22.86) (end 14.605 -20.955) (width 0.3048) (layer "B.Cu") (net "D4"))
 (segment (start 25.4 -15.24) (end 25.4 -21.59) (width 0.3048) (layer "B.Cu") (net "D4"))
 (segment (start 14.605 -20.955) (end 14.605 -20.32) (width 0.3048) (layer "B.Cu") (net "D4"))
 (segment (start 24.13 -12.7) (end 24.13 -13.97) (width 0.3048) (layer "B.Cu") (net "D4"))
 (segment (start 24.13 -22.86) (end 16.51 -22.86) (width 0.3048) (layer "B.Cu") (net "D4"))
 (segment (start 24.13 -13.97) (end 25.4 -15.24) (width 0.3048) (layer "B.Cu") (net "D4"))
 (segment (start 24.13 -12.7) (end 24.13 -10.16) (width 0.6096) (layer "B.Cu") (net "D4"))
 (segment (start 25.4 -21.59) (end 24.13 -22.86) (width 0.3048) (layer "B.Cu") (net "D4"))
 (segment (start 34.29 -12.7) (end 34.29 -10.16) (width 0.6096) (layer "B.Cu") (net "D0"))
 (segment (start 34.29 -10.16) (end 36.83 -7.62) (width 0.6096) (layer "B.Cu") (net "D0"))
 (segment (start 31.75 -12.7) (end 31.75 -10.16) (width 0.6096) (layer "B.Cu") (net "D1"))
 (segment (start 31.75 -10.16) (end 34.29 -7.62) (width 0.6096) (layer "B.Cu") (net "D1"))
 (segment (start 29.21 -10.16) (end 31.75 -7.62) (width 0.6096) (layer "B.Cu") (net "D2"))
 (segment (start 29.21 -12.7) (end 29.21 -10.16) (width 0.6096) (layer "B.Cu") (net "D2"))
 (segment (start 26.67 -10.16) (end 29.21 -7.62) (width 0.6096) (layer "B.Cu") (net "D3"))
 (segment (start 26.67 -12.7) (end 26.67 -10.16) (width 0.6096) (layer "B.Cu") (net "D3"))
 (segment (start 23.8125 -16.8275) (end 20.0025 -16.8275) (width 0.6096) (layer "F.Cu") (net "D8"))
 (segment (start 26.67 -20.32) (end 26.67 -19.685) (width 0.6096) (layer "F.Cu") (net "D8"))
 (segment (start 20.0025 -16.8275) (end 16.51 -13.335) (width 0.6096) (layer "F.Cu") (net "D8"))
 (segment (start 26.67 -19.685) (end 23.8125 -16.8275) (width 0.6096) (layer "F.Cu") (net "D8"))
 (via (at 16.51 -13.335) (size 0.9556) (drill 0.6) (layers "F.Cu" "B.Cu") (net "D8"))
 (segment (start 16.51 -13.335) (end 16.51 -7.62) (width 0.6096) (layer "B.Cu") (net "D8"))
 (segment (start 20.6375 -15.875) (end 16.1925 -11.43) (width 0.6096) (layer "F.Cu") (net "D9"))
 (segment (start 31.75 -20.32) (end 31.75 -19.685) (width 0.6096) (layer "F.Cu") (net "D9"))
 (segment (start 27.94 -15.875) (end 20.6375 -15.875) (width 0.6096) (layer "F.Cu") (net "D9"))
 (segment (start 16.1925 -11.43) (end 14.9225 -11.43) (width 0.6096) (layer "F.Cu") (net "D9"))
 (segment (start 31.75 -19.685) (end 27.94 -15.875) (width 0.6096) (layer "F.Cu") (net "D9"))
 (via (at 14.9225 -11.43) (size 0.9556) (drill 0.6) (layers "F.Cu" "B.Cu") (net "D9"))
 (segment (start 14.9225 -11.43) (end 14.9225 -8.5725) (width 0.6096) (layer "B.Cu") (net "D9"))
 (segment (start 14.9225 -8.5725) (end 13.97 -7.62) (width 0.6096) (layer "B.Cu") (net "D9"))
 (segment (start 34.29 -19.685) (end 29.5275 -14.9225) (width 0.6096) (layer "F.Cu") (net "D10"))
 (segment (start 21.2725 -14.9225) (end 16.51 -10.16) (width 0.6096) (layer "F.Cu") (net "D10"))
 (segment (start 29.5275 -14.9225) (end 21.2725 -14.9225) (width 0.6096) (layer "F.Cu") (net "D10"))
 (segment (start 13.97 -10.16) (end 11.43 -7.62) (width 0.6096) (layer "F.Cu") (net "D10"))
 (segment (start 16.51 -10.16) (end 13.97 -10.16) (width 0.6096) (layer "F.Cu") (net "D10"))
 (segment (start 34.29 -20.32) (end 34.29 -19.685) (width 0.6096) (layer "F.Cu") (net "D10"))
 (segment (start 24.13 -19.685) (end 22.5425 -18.0975) (width 0.6096) (layer "F.Cu") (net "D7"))
 (segment (start 22.5425 -18.0975) (end 20.32 -18.0975) (width 0.6096) (layer "F.Cu") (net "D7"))
 (segment (start 24.13 -20.32) (end 24.13 -19.685) (width 0.6096) (layer "F.Cu") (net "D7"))
 (via (at 20.32 -18.0975) (size 0.9556) (drill 0.6) (layers "F.Cu" "B.Cu") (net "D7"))
 (segment (start 18.415 -16.1925) (end 18.415 -8.255) (width 0.6096) (layer "B.Cu") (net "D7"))
 (segment (start 20.32 -18.0975) (end 18.415 -16.1925) (width 0.6096) (layer "B.Cu") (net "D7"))
 (segment (start 18.415 -8.255) (end 19.05 -7.62) (width 0.6096) (layer "B.Cu") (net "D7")))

